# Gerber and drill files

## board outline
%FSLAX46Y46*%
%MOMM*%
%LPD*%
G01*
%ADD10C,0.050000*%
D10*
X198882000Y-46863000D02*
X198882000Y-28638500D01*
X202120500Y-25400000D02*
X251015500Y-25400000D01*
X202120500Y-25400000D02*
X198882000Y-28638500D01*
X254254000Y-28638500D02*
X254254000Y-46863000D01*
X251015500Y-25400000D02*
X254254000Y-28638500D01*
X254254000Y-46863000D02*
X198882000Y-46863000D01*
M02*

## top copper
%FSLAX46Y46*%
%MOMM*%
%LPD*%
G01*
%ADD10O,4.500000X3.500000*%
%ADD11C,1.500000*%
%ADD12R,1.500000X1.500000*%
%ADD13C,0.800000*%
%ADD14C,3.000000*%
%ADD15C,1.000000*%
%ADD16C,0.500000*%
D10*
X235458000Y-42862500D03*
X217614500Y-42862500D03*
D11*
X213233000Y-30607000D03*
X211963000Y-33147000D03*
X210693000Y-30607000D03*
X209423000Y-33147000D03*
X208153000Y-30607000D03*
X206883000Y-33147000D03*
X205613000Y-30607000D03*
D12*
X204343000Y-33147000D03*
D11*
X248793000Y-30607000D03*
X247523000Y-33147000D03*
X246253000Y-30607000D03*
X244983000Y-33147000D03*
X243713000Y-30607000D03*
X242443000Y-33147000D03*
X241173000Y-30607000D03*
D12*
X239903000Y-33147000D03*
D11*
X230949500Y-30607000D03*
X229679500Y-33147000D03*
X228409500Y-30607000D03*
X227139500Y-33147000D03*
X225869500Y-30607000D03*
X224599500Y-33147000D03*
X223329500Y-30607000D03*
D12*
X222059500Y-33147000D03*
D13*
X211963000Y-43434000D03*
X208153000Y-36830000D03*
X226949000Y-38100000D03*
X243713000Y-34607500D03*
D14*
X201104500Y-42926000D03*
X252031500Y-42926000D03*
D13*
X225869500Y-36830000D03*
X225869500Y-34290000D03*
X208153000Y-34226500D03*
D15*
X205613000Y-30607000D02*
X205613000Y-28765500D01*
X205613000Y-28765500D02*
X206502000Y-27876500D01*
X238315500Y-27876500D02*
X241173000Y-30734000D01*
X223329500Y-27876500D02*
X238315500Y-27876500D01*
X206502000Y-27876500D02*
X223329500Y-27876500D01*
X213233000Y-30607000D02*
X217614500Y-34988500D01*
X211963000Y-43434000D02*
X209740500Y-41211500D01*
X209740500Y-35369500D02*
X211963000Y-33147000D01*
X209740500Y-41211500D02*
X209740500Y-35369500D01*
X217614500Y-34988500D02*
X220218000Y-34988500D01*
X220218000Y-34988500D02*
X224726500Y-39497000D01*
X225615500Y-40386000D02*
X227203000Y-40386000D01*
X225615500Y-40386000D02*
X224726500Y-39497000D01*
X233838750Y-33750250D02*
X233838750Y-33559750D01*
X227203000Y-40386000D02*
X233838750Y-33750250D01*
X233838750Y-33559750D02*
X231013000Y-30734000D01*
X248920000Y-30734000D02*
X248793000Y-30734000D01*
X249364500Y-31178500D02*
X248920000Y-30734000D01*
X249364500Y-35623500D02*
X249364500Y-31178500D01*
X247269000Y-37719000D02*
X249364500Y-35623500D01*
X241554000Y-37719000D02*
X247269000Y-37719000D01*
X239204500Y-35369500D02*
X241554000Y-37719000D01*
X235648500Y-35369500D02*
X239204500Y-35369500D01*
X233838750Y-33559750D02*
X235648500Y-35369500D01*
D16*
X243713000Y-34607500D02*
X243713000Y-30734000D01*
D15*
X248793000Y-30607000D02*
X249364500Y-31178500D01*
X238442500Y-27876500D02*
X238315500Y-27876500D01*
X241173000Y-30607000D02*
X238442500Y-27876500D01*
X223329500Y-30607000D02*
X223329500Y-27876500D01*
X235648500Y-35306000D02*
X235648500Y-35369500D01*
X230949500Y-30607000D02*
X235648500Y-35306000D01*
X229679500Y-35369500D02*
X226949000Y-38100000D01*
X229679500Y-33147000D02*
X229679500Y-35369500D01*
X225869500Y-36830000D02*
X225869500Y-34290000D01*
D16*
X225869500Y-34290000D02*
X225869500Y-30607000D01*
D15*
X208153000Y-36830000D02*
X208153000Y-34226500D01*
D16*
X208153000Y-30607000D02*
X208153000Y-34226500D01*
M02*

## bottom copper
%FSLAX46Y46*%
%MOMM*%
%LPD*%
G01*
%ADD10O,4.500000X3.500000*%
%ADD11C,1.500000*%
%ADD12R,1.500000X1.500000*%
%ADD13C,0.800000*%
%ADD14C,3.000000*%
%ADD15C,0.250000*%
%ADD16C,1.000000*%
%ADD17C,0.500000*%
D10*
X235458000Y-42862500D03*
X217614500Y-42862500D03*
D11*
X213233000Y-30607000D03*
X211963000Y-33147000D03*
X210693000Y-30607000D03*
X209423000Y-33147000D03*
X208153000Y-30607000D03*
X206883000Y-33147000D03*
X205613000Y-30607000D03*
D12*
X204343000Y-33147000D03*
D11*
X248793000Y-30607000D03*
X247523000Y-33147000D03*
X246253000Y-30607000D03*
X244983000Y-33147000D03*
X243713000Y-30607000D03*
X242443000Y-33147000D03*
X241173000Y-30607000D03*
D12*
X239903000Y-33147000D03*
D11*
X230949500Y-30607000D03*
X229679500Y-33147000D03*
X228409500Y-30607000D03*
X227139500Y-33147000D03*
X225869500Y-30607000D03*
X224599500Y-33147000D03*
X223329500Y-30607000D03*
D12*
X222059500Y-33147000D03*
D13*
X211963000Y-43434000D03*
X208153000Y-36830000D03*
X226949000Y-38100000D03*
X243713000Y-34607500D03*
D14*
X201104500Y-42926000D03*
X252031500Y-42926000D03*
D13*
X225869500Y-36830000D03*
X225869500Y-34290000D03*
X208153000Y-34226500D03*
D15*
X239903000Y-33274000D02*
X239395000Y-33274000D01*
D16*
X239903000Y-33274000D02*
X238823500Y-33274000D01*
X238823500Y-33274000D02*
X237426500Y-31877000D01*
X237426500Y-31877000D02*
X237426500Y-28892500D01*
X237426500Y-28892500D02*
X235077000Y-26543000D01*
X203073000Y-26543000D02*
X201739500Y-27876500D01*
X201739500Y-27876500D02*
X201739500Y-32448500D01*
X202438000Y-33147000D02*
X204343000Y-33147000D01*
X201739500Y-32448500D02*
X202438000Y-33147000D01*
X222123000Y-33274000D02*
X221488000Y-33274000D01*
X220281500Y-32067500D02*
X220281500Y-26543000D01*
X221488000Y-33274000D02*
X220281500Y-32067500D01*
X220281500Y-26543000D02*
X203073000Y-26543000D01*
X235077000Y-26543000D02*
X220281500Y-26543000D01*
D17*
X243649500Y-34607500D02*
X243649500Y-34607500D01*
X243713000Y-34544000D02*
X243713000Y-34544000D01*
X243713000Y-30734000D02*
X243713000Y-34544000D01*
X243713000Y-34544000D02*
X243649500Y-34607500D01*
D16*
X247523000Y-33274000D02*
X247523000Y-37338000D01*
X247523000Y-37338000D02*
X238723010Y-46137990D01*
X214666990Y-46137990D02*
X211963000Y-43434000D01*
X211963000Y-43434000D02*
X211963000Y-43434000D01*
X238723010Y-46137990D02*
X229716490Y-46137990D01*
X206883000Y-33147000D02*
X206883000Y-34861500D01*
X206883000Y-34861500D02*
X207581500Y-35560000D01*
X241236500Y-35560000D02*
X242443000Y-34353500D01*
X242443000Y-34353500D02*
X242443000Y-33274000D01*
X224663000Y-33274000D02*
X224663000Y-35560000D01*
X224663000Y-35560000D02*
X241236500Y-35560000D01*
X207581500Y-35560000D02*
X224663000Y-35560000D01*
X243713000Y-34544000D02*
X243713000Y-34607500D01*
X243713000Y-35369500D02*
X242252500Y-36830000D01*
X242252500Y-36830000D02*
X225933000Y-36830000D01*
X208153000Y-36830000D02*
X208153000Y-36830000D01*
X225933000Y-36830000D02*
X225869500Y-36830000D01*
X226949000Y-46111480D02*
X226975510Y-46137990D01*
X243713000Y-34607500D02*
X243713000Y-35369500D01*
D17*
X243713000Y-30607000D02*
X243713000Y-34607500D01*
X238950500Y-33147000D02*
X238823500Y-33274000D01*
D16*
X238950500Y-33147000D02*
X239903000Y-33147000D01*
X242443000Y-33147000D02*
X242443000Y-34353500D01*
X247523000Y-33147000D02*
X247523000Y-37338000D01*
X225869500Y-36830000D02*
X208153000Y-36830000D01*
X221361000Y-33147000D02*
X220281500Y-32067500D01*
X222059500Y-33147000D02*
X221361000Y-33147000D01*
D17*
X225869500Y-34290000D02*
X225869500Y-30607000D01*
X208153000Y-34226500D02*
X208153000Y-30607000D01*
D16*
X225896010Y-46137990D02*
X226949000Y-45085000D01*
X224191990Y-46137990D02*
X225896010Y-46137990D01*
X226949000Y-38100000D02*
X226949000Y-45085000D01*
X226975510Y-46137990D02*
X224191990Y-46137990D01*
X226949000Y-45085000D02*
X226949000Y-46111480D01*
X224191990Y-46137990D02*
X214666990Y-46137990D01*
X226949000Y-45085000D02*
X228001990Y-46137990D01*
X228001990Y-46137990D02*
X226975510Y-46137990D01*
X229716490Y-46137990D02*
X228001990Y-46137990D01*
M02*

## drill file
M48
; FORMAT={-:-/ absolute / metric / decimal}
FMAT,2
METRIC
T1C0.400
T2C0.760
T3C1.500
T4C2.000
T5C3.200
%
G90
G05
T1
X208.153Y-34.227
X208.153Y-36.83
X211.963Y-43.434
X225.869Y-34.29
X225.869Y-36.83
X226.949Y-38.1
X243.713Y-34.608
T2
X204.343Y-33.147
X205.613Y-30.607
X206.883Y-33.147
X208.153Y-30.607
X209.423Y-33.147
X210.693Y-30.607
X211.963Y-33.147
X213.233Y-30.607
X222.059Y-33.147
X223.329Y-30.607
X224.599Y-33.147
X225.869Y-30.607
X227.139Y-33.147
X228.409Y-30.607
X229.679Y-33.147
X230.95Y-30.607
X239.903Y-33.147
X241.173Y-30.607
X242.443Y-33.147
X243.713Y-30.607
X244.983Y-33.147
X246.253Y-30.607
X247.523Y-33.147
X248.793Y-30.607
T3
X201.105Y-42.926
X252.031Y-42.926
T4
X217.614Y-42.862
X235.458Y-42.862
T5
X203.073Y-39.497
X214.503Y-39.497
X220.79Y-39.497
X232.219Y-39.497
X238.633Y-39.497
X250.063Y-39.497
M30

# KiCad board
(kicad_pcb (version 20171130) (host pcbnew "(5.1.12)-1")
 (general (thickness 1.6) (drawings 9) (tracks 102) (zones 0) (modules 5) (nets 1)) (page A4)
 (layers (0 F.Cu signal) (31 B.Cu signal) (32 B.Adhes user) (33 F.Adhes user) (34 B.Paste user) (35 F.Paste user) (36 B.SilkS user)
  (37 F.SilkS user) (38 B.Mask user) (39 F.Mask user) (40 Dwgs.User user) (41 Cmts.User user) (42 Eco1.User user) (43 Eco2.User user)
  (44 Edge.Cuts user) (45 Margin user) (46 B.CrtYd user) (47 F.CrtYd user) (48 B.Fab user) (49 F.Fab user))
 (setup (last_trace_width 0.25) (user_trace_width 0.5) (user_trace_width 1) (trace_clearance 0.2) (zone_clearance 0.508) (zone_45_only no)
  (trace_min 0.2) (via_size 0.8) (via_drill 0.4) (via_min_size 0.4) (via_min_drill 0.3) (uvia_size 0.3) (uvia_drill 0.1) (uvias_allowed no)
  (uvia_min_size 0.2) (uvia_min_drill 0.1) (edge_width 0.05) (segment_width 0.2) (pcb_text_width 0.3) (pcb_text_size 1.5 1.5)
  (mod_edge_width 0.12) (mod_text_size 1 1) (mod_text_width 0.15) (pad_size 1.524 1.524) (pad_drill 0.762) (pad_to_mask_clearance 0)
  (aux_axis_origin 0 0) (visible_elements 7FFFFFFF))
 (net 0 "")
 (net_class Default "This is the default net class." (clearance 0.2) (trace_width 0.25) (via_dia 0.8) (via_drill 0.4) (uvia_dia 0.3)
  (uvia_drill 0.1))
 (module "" (layer F.Cu) (at 232.918 42.8625)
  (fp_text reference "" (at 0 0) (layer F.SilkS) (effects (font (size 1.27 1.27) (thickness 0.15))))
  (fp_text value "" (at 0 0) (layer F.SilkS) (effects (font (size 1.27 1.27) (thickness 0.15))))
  (pad 1 thru_hole oval (at 2.54 0) (size 4.5 3.5) (drill 2) (layers *.Cu *.Mask)))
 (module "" (layer F.Cu) (at 215.0745 42.8625)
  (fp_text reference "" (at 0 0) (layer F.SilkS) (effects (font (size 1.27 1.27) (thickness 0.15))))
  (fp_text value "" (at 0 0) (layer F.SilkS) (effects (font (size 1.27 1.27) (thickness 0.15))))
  (pad 1 thru_hole oval (at 2.54 0) (size 4.5 3.5) (drill 2) (layers *.Cu *.Mask)))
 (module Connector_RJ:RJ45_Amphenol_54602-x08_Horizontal (layer F.Cu) (at 204.343 33.147)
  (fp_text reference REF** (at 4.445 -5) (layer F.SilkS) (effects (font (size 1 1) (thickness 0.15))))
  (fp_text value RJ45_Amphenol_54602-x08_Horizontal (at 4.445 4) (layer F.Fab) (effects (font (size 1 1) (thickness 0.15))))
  (pad 8 thru_hole circle (at 8.89 -2.54) (size 1.5 1.5) (drill 0.76) (layers *.Cu *.Mask))
  (pad 7 thru_hole circle (at 7.62 0) (size 1.5 1.5) (drill 0.76) (layers *.Cu *.Mask))
  (pad 6 thru_hole circle (at 6.35 -2.54) (size 1.5 1.5) (drill 0.76) (layers *.Cu *.Mask))
  (pad 5 thru_hole circle (at 5.08 0) (size 1.5 1.5) (drill 0.76) (layers *.Cu *.Mask))
  (pad 4 thru_hole circle (at 3.81 -2.54) (size 1.5 1.5) (drill 0.76) (layers *.Cu *.Mask))
  (pad 3 thru_hole circle (at 2.54 0) (size 1.5 1.5) (drill 0.76) (layers *.Cu *.Mask))
  (pad 2 thru_hole circle (at 1.27 -2.54) (size 1.5 1.5) (drill 0.76) (layers *.Cu *.Mask))
  (pad 1 thru_hole rect (at 0 0) (size 1.5 1.5) (drill 0.76) (layers *.Cu *.Mask))
  (pad "" np_thru_hole circle (at -1.27 6.35) (size 3.2 3.2) (drill 3.2) (layers *.Cu *.Mask))
  (pad "" np_thru_hole circle (at 10.16 6.35) (size 3.2 3.2) (drill 3.2) (layers *.Cu *.Mask)))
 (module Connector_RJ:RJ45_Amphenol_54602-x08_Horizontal (layer F.Cu) (at 239.903 33.147)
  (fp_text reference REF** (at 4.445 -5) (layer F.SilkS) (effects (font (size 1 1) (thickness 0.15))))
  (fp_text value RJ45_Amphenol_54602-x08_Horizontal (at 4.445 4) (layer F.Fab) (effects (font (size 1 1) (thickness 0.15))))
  (pad 8 thru_hole circle (at 8.89 -2.54) (size 1.5 1.5) (drill 0.76) (layers *.Cu *.Mask))
  (pad 7 thru_hole circle (at 7.62 0) (size 1.5 1.5) (drill 0.76) (layers *.Cu *.Mask))
  (pad 6 thru_hole circle (at 6.35 -2.54) (size 1.5 1.5) (drill 0.76) (layers *.Cu *.Mask))
  (pad 5 thru_hole circle (at 5.08 0) (size 1.5 1.5) (drill 0.76) (layers *.Cu *.Mask))
  (pad 4 thru_hole circle (at 3.81 -2.54) (size 1.5 1.5) (drill 0.76) (layers *.Cu *.Mask))
  (pad 3 thru_hole circle (at 2.54 0) (size 1.5 1.5) (drill 0.76) (layers *.Cu *.Mask))
  (pad 2 thru_hole circle (at 1.27 -2.54) (size 1.5 1.5) (drill 0.76) (layers *.Cu *.Mask))
  (pad 1 thru_hole rect (at 0 0) (size 1.5 1.5) (drill 0.76) (layers *.Cu *.Mask))
  (pad "" np_thru_hole circle (at -1.27 6.35) (size 3.2 3.2) (drill 3.2) (layers *.Cu *.Mask))
  (pad "" np_thru_hole circle (at 10.16 6.35) (size 3.2 3.2) (drill 3.2) (layers *.Cu *.Mask)))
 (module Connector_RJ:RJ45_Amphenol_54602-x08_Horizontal (layer F.Cu) (at 222.0595 33.147)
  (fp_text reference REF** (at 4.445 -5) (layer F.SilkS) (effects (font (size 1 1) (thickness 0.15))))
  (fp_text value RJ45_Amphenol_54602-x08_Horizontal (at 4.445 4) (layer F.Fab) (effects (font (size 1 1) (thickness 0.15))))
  (pad 8 thru_hole circle (at 8.89 -2.54) (size 1.5 1.5) (drill 0.76) (layers *.Cu *.Mask))
  (pad 7 thru_hole circle (at 7.62 0) (size 1.5 1.5) (drill 0.76) (layers *.Cu *.Mask))
  (pad 6 thru_hole circle (at 6.35 -2.54) (size 1.5 1.5) (drill 0.76) (layers *.Cu *.Mask))
  (pad 5 thru_hole circle (at 5.08 0) (size 1.5 1.5) (drill 0.76) (layers *.Cu *.Mask))
  (pad 4 thru_hole circle (at 3.81 -2.54) (size 1.5 1.5) (drill 0.76) (layers *.Cu *.Mask))
  (pad 3 thru_hole circle (at 2.54 0) (size 1.5 1.5) (drill 0.76) (layers *.Cu *.Mask))
  (pad 2 thru_hole circle (at 1.27 -2.54) (size 1.5 1.5) (drill 0.76) (layers *.Cu *.Mask))
  (pad 1 thru_hole rect (at 0 0) (size 1.5 1.5) (drill 0.76) (layers *.Cu *.Mask))
  (pad "" np_thru_hole circle (at -1.27 6.35) (size 3.2 3.2) (drill 3.2) (layers *.Cu *.Mask))
  (pad "" np_thru_hole circle (at 10.16 6.35) (size 3.2 3.2) (drill 3.2) (layers *.Cu *.Mask)))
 (gr_line (start 198.882 46.863) (end 198.882 28.6385) (layer Edge.Cuts) (width 0.05))
 (gr_line (start 202.1205 25.4) (end 251.0155 25.4) (layer Edge.Cuts) (width 0.05))
 (gr_line (start 202.1205 25.4) (end 198.882 28.6385) (layer Edge.Cuts) (width 0.05))
 (gr_line (start 254.254 28.6385) (end 254.254 46.863) (layer Edge.Cuts) (width 0.05))
 (gr_line (start 251.0155 25.4) (end 254.254 28.6385) (layer Edge.Cuts) (width 0.05))
 (gr_line (start 254.254 46.863) (end 198.882 46.863) (layer Edge.Cuts) (width 0.05))
 (segment (start 239.903 33.274) (end 239.395 33.274) (width 0.25) (layer B.Cu) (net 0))
 (segment (start 239.903 33.274) (end 238.8235 33.274) (width 1) (layer B.Cu) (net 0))
 (segment (start 238.8235 33.274) (end 237.4265 31.877) (width 1) (layer B.Cu) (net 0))
 (segment (start 237.4265 31.877) (end 237.4265 28.8925) (width 1) (layer B.Cu) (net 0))
 (segment (start 237.4265 28.8925) (end 235.077 26.543) (width 1) (layer B.Cu) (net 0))
 (segment (start 203.073 26.543) (end 201.7395 27.8765) (width 1) (layer B.Cu) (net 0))
 (segment (start 201.7395 27.8765) (end 201.7395 32.4485) (width 1) (layer B.Cu) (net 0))
 (segment (start 202.438 33.147) (end 204.343 33.147) (width 1) (layer B.Cu) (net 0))
 (segment (start 201.7395 32.4485) (end 202.438 33.147) (width 1) (layer B.Cu) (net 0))
 (segment (start 222.123 33.274) (end 221.488 33.274) (width 1) (layer B.Cu) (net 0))
 (segment (start 220.2815 32.0675) (end 220.2815 26.543) (width 1) (layer B.Cu) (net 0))
 (segment (start 221.488 33.274) (end 220.2815 32.0675) (width 1) (layer B.Cu) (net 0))
 (segment (start 220.2815 26.543) (end 203.073 26.543) (width 1) (layer B.Cu) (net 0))
 (segment (start 235.077 26.543) (end 220.2815 26.543) (width 1) (layer B.Cu) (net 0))
 (segment (start 205.613 30.607) (end 205.613 28.7655) (width 1) (layer F.Cu) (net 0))
 (segment (start 205.613 28.7655) (end 206.502 27.8765) (width 1) (layer F.Cu) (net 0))
 (segment (start 238.3155 27.8765) (end 241.173 30.734) (width 1) (layer F.Cu) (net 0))
 (segment (start 223.3295 27.8765) (end 238.3155 27.8765) (width 1) (layer F.Cu) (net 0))
 (segment (start 206.502 27.8765) (end 223.3295 27.8765) (width 1) (layer F.Cu) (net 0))
 (segment (start 243.6495 34.6075) (end 243.6495 34.6075) (width 0.5) (layer B.Cu) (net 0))
 (segment (start 243.713 34.544) (end 243.713 34.544) (width 0.5) (layer B.Cu) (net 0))
 (segment (start 243.713 30.734) (end 243.713 34.544) (width 0.5) (layer B.Cu) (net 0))
 (segment (start 243.713 34.544) (end 243.6495 34.6075) (width 0.5) (layer B.Cu) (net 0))
 (segment (start 247.523 33.274) (end 247.523 37.338) (width 1) (layer B.Cu) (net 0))
 (segment (start 247.523 37.338) (end 238.72301 46.13799) (width 1) (layer B.Cu) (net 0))
 (segment (start 214.66699 46.13799) (end 211.963 43.434) (width 1) (layer B.Cu) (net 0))
 (segment (start 211.963 43.434) (end 211.963 43.434) (width 1) (layer B.Cu) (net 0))
 (via (at 211.963 43.434) (size 0.8) (drill 0.4) (layers F.Cu B.Cu) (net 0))
 (segment (start 238.72301 46.13799) (end 229.71649 46.13799) (width 1) (layer B.Cu) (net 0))
 (segment (start 206.883 33.147) (end 206.883 34.8615) (width 1) (layer B.Cu) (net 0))
 (segment (start 206.883 34.8615) (end 207.5815 35.56) (width 1) (layer B.Cu) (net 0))
 (segment (start 241.2365 35.56) (end 242.443 34.3535) (width 1) (layer B.Cu) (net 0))
 (segment (start 242.443 34.3535) (end 242.443 33.274) (width 1) (layer B.Cu) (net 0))
 (segment (start 224.663 33.274) (end 224.663 35.56) (width 1) (layer B.Cu) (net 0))
 (segment (start 224.663 35.56) (end 241.2365 35.56) (width 1) (layer B.Cu) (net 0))
 (segment (start 207.5815 35.56) (end 224.663 35.56) (width 1) (layer B.Cu) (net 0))
 (segment (start 243.713 34.544) (end 243.713 34.6075) (width 1) (layer B.Cu) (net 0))
 (segment (start 243.713 35.3695) (end 242.2525 36.83) (width 1) (layer B.Cu) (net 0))
 (segment (start 242.2525 36.83) (end 225.933 36.83) (width 1) (layer B.Cu) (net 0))
 (segment (start 208.153 36.83) (end 208.153 36.83) (width 1) (layer B.Cu) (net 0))
 (via (at 208.153 36.83) (size 0.8) (drill 0.4) (layers F.Cu B.Cu) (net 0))
 (segment (start 225.933 36.83) (end 225.8695 36.83) (width 1) (layer B.Cu) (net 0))
 (segment (start 213.233 30.607) (end 217.6145 34.9885) (width 1) (layer F.Cu) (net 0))
 (segment (start 211.963 43.434) (end 209.7405 41.2115) (width 1) (layer F.Cu) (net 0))
 (segment (start 209.7405 35.3695) (end 211.963 33.147) (width 1) (layer F.Cu) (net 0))
 (segment (start 209.7405 41.2115) (end 209.7405 35.3695) (width 1) (layer F.Cu) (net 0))
 (segment (start 217.6145 34.9885) (end 220.218 34.9885) (width 1) (layer F.Cu) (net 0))
 (segment (start 220.218 34.9885) (end 224.7265 39.497) (width 1) (layer F.Cu) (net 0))
 (via (at 226.949 38.1) (size 0.8) (drill 0.4) (layers F.Cu B.Cu) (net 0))
 (segment (start 225.6155 40.386) (end 227.203 40.386) (width 1) (layer F.Cu) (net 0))
 (segment (start 225.6155 40.386) (end 224.7265 39.497) (width 1) (layer F.Cu) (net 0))
 (segment (start 233.83875 33.75025) (end 233.83875 33.55975) (width 1) (layer F.Cu) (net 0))
 (segment (start 227.203 40.386) (end 233.83875 33.75025) (width 1) (layer F.Cu) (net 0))
 (segment (start 233.83875 33.55975) (end 231.013 30.734) (width 1) (layer F.Cu) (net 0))
 (segment (start 248.92 30.734) (end 248.793 30.734) (width 1) (layer F.Cu) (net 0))
 (segment (start 249.3645 31.1785) (end 248.92 30.734) (width 1) (layer F.Cu) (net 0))
 (segment (start 249.3645 35.6235) (end 249.3645 31.1785) (width 1) (layer F.Cu) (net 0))
 (segment (start 247.269 37.719) (end 249.3645 35.6235) (width 1) (layer F.Cu) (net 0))
 (segment (start 241.554 37.719) (end 247.269 37.719) (width 1) (layer F.Cu) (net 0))
 (segment (start 239.2045 35.3695) (end 241.554 37.719) (width 1) (layer F.Cu) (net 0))
 (segment (start 235.6485 35.3695) (end 239.2045 35.3695) (width 1) (layer F.Cu) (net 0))
 (segment (start 233.83875 33.55975) (end 235.6485 35.3695) (width 1) (layer F.Cu) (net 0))
 (segment (start 226.949 46.11148) (end 226.97551 46.13799) (width 1) (layer B.Cu) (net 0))
 (segment (start 243.713 34.6075) (end 243.713 35.3695) (width 1) (layer B.Cu) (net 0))
 (via (at 243.713 34.6075) (size 0.8) (drill 0.4) (layers F.Cu B.Cu) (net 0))
 (segment (start 243.713 34.6075) (end 243.713 30.734) (width 0.5) (layer F.Cu) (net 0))
 (via (at 201.1045 42.926) (size 3) (drill 1.5) (layers F.Cu B.Cu) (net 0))
 (via (at 252.0315 42.926) (size 3) (drill 1.5) (layers F.Cu B.Cu) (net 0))
 (segment (start 248.793 30.607) (end 249.3645 31.1785) (width 1) (layer F.Cu) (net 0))
 (segment (start 243.713 30.607) (end 243.713 34.6075) (width 0.5) (layer B.Cu) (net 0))
 (segment (start 238.9505 33.147) (end 238.8235 33.274) (width 0.5) (layer B.Cu) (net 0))
 (segment (start 238.9505 33.147) (end 239.903 33.147) (width 1) (layer B.Cu) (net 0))
 (segment (start 238.4425 27.8765) (end 238.3155 27.8765) (width 1) (layer F.Cu) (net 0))
 (segment (start 241.173 30.607) (end 238.4425 27.8765) (width 1) (layer F.Cu) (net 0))
 (segment (start 242.443 33.147) (end 242.443 34.3535) (width 1) (layer B.Cu) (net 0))
 (segment (start 247.523 33.147) (end 247.523 37.338) (width 1) (layer B.Cu) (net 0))
 (segment (start 225.8695 36.83) (end 208.153 36.83) (width 1) (layer B.Cu) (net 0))
 (via (at 225.8695 36.83) (size 0.8) (drill 0.4) (layers F.Cu B.Cu) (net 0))
 (segment (start 223.3295 30.607) (end 223.3295 27.8765) (width 1) (layer F.Cu) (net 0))
 (segment (start 235.6485 35.306) (end 235.6485 35.3695) (width 1) (layer F.Cu) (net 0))
 (segment (start 230.9495 30.607) (end 235.6485 35.306) (width 1) (layer F.Cu) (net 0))
 (segment (start 229.6795 35.3695) (end 226.949 38.1) (width 1) (layer F.Cu) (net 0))
 (segment (start 229.6795 33.147) (end 229.6795 35.3695) (width 1) (layer F.Cu) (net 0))
 (segment (start 221.361 33.147) (end 220.2815 32.0675) (width 1) (layer B.Cu) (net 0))
 (segment (start 222.0595 33.147) (end 221.361 33.147) (width 1) (layer B.Cu) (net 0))
 (segment (start 225.8695 36.83) (end 225.8695 34.29) (width 1) (layer F.Cu) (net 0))
 (via (at 225.8695 34.29) (size 0.8) (drill 0.4) (layers F.Cu B.Cu) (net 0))
 (segment (start 225.8695 34.29) (end 225.8695 30.607) (width 0.5) (layer F.Cu) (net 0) (status 40000))
 (segment (start 225.8695 34.29) (end 225.8695 30.607) (width 0.5) (layer B.Cu) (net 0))
 (via (at 208.153 34.2265) (size 0.8) (drill 0.4) (layers F.Cu B.Cu) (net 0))
 (segment (start 208.153 36.83) (end 208.153 34.2265) (width 1) (layer F.Cu) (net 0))
 (segment (start 208.153 30.607) (end 208.153 34.2265) (width 0.5) (layer F.Cu) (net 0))
 (segment (start 208.153 34.2265) (end 208.153 30.607) (width 0.5) (layer B.Cu) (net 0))
 (segment (start 225.89601 46.13799) (end 226.949 45.085) (width 1) (layer B.Cu) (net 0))
 (segment (start 224.19199 46.13799) (end 225.89601 46.13799) (width 1) (layer B.Cu) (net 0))
 (segment (start 226.949 38.1) (end 226.949 45.085) (width 1) (layer B.Cu) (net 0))
 (segment (start 226.97551 46.13799) (end 224.19199 46.13799) (width 1) (layer B.Cu) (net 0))
 (segment (start 226.949 45.085) (end 226.949 46.11148) (width 1) (layer B.Cu) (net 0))
 (segment (start 224.19199 46.13799) (end 214.66699 46.13799) (width 1) (layer B.Cu) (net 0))
 (segment (start 226.949 45.085) (end 228.00199 46.13799) (width 1) (layer B.Cu) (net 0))
 (segment (start 228.00199 46.13799) (end 226.97551 46.13799) (width 1) (layer B.Cu) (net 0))
 (segment (start 229.71649 46.13799) (end 228.00199 46.13799) (width 1) (layer B.Cu) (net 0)))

